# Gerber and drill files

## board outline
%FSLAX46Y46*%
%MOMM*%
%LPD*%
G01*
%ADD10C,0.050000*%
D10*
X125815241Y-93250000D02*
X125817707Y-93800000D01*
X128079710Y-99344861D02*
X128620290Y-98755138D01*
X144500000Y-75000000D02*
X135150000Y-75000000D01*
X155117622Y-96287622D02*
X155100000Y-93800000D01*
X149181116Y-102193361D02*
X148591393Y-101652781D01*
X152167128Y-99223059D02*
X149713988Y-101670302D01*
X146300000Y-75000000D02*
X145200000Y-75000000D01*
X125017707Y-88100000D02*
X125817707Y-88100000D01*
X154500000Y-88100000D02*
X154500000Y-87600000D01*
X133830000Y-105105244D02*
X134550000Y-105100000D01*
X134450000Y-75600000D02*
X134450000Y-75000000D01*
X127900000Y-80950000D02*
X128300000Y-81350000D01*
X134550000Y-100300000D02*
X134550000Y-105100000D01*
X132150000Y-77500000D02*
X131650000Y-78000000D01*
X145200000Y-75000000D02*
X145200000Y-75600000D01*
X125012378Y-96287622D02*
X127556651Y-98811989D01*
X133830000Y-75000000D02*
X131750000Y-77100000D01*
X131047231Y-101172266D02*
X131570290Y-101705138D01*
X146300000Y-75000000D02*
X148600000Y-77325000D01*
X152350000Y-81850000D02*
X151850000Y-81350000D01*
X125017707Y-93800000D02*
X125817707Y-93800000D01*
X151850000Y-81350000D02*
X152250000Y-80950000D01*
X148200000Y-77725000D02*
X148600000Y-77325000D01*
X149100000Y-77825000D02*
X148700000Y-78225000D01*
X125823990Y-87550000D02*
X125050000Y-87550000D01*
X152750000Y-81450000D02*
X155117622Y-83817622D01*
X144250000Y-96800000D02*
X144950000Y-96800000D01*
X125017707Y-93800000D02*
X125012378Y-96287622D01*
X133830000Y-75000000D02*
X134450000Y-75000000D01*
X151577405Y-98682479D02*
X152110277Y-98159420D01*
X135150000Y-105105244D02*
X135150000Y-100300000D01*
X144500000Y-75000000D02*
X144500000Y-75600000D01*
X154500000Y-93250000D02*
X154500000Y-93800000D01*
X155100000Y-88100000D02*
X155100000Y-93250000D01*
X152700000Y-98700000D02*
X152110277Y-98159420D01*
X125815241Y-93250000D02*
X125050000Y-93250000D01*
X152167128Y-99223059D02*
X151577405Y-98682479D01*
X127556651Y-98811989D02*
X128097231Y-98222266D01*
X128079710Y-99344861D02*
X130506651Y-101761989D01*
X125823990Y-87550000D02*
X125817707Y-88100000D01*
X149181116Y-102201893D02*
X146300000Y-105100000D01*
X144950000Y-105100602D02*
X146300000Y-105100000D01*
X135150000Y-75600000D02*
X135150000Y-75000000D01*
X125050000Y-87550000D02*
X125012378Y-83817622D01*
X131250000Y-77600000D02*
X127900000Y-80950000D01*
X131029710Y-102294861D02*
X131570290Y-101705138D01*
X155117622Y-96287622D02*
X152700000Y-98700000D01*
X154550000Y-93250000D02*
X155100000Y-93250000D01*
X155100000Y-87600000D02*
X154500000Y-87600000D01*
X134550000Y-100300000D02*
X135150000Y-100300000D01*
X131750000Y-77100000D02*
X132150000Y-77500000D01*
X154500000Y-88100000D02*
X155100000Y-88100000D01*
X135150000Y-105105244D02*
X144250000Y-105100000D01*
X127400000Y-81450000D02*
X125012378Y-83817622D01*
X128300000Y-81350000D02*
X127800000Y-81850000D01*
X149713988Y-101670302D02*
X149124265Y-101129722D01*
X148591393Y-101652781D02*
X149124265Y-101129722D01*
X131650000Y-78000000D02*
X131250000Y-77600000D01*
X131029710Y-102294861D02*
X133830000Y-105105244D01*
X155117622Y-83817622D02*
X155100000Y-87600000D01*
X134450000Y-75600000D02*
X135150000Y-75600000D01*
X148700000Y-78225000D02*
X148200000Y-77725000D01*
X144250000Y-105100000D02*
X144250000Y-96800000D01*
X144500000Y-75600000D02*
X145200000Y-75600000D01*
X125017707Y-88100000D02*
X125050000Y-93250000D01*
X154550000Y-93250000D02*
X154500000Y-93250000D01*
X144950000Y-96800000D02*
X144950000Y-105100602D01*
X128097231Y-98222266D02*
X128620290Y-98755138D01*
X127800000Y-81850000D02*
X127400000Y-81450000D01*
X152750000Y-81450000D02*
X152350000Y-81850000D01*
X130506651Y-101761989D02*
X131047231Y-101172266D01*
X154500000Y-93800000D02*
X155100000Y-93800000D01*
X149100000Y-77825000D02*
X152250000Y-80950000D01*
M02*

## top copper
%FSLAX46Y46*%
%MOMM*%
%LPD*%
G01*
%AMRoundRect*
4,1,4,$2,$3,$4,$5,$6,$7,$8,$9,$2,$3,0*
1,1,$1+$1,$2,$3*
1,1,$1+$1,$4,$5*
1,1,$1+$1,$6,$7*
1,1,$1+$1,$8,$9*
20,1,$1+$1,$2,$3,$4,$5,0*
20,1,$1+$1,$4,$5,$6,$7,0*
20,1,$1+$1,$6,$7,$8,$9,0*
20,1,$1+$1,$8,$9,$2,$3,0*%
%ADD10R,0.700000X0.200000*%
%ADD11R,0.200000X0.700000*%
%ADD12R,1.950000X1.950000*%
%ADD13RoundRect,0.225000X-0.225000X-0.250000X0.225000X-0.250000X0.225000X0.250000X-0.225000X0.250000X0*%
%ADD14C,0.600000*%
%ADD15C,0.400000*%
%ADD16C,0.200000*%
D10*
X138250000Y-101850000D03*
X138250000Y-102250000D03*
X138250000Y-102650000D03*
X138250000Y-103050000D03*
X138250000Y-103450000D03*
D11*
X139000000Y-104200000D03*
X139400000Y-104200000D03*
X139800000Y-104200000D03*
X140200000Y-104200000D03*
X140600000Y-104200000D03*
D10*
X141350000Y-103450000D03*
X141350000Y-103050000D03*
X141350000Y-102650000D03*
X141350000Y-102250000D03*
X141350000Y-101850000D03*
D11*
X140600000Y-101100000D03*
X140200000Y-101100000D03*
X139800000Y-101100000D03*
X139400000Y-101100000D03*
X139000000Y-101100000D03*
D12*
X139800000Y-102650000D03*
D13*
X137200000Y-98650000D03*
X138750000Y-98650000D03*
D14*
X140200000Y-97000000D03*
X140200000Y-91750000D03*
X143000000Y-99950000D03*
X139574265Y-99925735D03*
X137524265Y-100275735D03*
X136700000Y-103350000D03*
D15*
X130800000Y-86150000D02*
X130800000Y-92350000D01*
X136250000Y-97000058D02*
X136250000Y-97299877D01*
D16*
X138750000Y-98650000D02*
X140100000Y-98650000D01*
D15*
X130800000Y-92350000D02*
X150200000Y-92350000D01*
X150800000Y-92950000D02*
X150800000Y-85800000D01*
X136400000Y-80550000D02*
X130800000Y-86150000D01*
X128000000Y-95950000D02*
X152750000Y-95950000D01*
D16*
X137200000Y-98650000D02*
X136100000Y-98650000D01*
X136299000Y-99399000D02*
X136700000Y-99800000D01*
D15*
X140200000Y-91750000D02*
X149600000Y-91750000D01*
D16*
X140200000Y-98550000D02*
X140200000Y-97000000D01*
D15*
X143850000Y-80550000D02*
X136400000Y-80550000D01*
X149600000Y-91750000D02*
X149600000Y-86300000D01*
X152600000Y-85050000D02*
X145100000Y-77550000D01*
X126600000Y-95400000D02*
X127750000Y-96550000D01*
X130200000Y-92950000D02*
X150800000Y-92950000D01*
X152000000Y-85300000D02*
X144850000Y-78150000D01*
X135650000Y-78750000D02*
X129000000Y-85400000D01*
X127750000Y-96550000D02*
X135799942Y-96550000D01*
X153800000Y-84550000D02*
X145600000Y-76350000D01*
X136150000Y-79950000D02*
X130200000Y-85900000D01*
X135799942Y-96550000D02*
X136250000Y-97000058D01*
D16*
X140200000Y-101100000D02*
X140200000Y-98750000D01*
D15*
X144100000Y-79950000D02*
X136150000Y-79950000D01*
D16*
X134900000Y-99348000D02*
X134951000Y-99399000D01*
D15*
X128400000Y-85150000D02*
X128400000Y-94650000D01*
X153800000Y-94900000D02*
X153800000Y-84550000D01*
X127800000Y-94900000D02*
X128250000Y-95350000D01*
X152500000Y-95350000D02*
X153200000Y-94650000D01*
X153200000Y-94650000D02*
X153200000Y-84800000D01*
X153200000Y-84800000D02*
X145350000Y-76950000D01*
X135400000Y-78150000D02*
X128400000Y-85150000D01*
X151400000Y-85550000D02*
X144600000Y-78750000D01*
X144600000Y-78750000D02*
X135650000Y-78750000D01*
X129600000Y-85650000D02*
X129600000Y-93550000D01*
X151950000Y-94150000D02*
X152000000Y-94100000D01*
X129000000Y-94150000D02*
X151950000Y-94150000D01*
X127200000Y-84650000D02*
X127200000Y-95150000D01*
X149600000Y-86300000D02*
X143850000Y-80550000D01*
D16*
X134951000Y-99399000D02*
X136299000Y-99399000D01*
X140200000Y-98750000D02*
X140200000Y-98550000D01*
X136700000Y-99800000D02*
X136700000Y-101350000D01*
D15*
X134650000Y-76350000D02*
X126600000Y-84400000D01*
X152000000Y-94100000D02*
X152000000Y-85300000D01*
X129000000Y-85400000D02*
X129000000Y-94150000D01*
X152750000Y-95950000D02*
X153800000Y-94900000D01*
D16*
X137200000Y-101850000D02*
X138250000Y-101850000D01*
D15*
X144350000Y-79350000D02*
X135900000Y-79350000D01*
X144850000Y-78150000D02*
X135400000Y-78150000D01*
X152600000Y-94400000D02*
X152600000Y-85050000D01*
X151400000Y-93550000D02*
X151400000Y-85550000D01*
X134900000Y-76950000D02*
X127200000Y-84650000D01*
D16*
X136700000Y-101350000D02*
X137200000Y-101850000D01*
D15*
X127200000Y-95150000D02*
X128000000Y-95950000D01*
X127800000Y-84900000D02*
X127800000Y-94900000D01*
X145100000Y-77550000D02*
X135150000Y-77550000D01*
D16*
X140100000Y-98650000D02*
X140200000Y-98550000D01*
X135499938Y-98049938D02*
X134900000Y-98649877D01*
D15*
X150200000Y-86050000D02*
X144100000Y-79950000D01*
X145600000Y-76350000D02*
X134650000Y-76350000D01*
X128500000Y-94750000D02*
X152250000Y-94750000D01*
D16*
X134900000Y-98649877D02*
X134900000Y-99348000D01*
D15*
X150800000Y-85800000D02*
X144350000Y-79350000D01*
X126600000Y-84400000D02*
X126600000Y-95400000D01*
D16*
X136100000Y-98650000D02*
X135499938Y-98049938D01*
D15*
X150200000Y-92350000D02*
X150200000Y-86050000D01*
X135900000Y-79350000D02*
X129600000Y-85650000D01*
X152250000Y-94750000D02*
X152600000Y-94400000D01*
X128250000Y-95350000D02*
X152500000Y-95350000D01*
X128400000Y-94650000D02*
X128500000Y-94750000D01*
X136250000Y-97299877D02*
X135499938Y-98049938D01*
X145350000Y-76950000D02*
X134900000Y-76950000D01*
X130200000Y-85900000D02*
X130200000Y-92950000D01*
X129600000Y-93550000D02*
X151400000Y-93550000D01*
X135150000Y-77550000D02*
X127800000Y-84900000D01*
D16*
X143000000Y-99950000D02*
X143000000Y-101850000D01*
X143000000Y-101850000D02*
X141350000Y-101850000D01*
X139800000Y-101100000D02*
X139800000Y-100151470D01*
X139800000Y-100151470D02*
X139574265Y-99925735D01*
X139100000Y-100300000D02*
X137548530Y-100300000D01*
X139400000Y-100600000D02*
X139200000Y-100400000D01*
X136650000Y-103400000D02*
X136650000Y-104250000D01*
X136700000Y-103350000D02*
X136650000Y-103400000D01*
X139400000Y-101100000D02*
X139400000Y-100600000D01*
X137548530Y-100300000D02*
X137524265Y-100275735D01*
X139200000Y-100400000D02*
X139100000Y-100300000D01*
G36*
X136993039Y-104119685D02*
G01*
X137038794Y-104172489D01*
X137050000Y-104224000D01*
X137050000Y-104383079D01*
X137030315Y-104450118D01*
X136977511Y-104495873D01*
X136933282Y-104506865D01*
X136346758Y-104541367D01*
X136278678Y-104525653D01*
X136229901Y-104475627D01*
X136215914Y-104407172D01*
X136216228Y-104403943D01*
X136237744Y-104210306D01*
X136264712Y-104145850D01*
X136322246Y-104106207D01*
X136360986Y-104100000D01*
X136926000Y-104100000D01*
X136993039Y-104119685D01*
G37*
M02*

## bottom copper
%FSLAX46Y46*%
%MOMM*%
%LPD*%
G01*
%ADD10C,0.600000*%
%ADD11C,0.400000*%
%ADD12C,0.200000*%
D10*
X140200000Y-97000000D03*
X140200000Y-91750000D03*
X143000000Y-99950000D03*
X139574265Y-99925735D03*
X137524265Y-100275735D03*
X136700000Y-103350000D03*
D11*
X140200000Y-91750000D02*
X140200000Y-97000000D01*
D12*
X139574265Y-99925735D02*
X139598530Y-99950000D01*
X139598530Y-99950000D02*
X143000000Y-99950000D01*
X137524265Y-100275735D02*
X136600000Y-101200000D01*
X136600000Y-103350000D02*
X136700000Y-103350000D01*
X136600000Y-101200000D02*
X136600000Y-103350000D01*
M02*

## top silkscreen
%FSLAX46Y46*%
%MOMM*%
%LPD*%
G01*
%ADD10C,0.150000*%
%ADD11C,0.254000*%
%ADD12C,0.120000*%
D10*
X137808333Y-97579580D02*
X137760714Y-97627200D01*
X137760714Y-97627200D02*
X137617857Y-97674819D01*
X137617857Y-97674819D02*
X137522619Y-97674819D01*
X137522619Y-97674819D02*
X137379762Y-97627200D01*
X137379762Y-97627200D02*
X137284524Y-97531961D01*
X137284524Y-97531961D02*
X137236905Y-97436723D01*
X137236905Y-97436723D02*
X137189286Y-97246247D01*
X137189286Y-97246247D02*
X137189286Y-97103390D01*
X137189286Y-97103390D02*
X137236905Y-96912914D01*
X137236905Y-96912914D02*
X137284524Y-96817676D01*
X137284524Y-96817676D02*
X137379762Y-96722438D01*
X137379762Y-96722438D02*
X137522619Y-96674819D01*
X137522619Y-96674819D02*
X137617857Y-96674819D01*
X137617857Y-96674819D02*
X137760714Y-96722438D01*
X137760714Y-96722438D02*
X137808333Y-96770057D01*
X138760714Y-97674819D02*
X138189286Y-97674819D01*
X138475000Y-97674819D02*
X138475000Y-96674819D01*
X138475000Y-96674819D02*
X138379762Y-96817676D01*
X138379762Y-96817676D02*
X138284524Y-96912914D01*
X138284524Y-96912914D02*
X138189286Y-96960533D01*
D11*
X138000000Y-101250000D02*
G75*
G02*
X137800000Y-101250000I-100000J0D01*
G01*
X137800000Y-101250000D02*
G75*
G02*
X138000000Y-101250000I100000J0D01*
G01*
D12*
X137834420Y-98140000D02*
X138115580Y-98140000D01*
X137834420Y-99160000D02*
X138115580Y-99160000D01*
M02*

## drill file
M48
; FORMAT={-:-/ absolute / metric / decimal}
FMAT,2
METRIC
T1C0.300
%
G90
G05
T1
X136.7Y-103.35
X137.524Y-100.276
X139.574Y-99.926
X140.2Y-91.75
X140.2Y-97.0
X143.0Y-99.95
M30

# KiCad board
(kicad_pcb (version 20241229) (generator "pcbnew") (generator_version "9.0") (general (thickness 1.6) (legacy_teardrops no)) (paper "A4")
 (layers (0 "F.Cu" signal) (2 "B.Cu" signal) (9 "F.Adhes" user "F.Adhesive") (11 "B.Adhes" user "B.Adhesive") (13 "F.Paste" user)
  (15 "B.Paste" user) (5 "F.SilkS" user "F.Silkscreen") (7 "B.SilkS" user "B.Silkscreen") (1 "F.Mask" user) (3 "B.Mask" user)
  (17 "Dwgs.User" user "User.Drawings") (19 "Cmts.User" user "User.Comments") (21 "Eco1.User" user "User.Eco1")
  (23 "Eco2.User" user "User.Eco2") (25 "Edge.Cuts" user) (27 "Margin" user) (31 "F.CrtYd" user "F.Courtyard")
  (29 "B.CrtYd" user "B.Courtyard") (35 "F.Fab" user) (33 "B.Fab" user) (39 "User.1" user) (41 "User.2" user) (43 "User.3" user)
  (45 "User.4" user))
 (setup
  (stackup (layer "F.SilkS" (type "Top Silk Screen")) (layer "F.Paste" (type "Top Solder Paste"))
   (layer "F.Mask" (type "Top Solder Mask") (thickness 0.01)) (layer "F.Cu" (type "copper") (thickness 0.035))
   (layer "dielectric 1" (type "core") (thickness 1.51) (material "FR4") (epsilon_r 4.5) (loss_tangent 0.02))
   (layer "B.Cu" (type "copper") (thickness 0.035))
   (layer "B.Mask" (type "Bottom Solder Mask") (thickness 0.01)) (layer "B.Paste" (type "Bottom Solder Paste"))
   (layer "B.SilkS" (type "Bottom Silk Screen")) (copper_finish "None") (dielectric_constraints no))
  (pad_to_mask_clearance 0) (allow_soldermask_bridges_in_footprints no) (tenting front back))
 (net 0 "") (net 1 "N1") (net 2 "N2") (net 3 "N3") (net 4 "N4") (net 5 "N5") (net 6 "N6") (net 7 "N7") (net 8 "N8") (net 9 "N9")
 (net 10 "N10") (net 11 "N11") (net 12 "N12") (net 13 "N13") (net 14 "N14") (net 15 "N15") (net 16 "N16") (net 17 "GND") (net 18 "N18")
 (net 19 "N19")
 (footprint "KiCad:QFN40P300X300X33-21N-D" (layer "F.Cu") (at 139.8 102.65)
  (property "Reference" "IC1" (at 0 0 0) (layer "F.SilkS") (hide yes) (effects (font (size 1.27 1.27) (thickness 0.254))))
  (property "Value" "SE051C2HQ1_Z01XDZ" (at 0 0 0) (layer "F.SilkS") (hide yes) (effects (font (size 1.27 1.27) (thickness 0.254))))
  (fp_circle (center -1.9 -1.4) (end -1.8 -1.4) (stroke (width 0.254) (type solid)) (fill no) (layer "F.SilkS"))
  (pad "1" smd rect (at -1.55 -0.8 90) (size 0.2 0.7) (layers "F.Cu" "F.Mask" "F.Paste") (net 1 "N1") (solder_mask_margin 0.04)
   (thermal_bridge_angle 45))
  (pad "2" smd rect (at -1.55 -0.4 90) (size 0.2 0.7) (layers "F.Cu" "F.Mask" "F.Paste") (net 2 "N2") (solder_mask_margin 0.04)
   (thermal_bridge_angle 45))
  (pad "3" smd rect (at -1.55 0 90) (size 0.2 0.7) (layers "F.Cu" "F.Mask" "F.Paste") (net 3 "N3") (solder_mask_margin 0.04)
   (thermal_bridge_angle 45))
  (pad "4" smd rect (at -1.55 0.4 90) (size 0.2 0.7) (layers "F.Cu" "F.Mask" "F.Paste") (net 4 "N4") (solder_mask_margin 0.04)
   (thermal_bridge_angle 45))
  (pad "5" smd rect (at -1.55 0.8 90) (size 0.2 0.7) (layers "F.Cu" "F.Mask" "F.Paste") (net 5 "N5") (solder_mask_margin 0.04)
   (thermal_bridge_angle 45))
  (pad "6" smd rect (at -0.8 1.55) (size 0.2 0.7) (layers "F.Cu" "F.Mask" "F.Paste") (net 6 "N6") (solder_mask_margin 0.04)
   (thermal_bridge_angle 45))
  (pad "7" smd rect (at -0.4 1.55) (size 0.2 0.7) (layers "F.Cu" "F.Mask" "F.Paste") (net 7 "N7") (solder_mask_margin 0.04)
   (thermal_bridge_angle 45))
  (pad "8" smd rect (at 0 1.55) (size 0.2 0.7) (layers "F.Cu" "F.Mask" "F.Paste") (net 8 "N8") (solder_mask_margin 0.04)
   (thermal_bridge_angle 45))
  (pad "9" smd rect (at 0.4 1.55) (size 0.2 0.7) (layers "F.Cu" "F.Mask" "F.Paste") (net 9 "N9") (solder_mask_margin 0.04)
   (thermal_bridge_angle 45))
  (pad "10" smd rect (at 0.8 1.55) (size 0.2 0.7) (layers "F.Cu" "F.Mask" "F.Paste") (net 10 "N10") (solder_mask_margin 0.04)
   (thermal_bridge_angle 45))
  (pad "11" smd rect (at 1.55 0.8 90) (size 0.2 0.7) (layers "F.Cu" "F.Mask" "F.Paste") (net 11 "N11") (solder_mask_margin 0.04)
   (thermal_bridge_angle 45))
  (pad "12" smd rect (at 1.55 0.4 90) (size 0.2 0.7) (layers "F.Cu" "F.Mask" "F.Paste") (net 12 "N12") (solder_mask_margin 0.04)
   (thermal_bridge_angle 45))
  (pad "13" smd rect (at 1.55 0 90) (size 0.2 0.7) (layers "F.Cu" "F.Mask" "F.Paste") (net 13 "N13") (solder_mask_margin 0.04)
   (thermal_bridge_angle 45))
  (pad "14" smd rect (at 1.55 -0.4 90) (size 0.2 0.7) (layers "F.Cu" "F.Mask" "F.Paste") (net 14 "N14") (solder_mask_margin 0.04)
   (thermal_bridge_angle 45))
  (pad "15" smd rect (at 1.55 -0.8 90) (size 0.2 0.7) (layers "F.Cu" "F.Mask" "F.Paste") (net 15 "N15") (solder_mask_margin 0.04)
   (thermal_bridge_angle 45))
  (pad "16" smd rect (at 0.8 -1.55) (size 0.2 0.7) (layers "F.Cu" "F.Mask" "F.Paste") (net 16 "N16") (solder_mask_margin 0.04)
   (thermal_bridge_angle 45))
  (pad "17" smd rect (at 0.4 -1.55) (size 0.2 0.7) (layers "F.Cu" "F.Mask" "F.Paste") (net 1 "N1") (solder_mask_margin 0.04)
   (thermal_bridge_angle 45))
  (pad "18" smd rect (at 0 -1.55) (size 0.2 0.7) (layers "F.Cu" "F.Mask" "F.Paste") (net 15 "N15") (solder_mask_margin 0.04)
   (thermal_bridge_angle 45))
  (pad "19" smd rect (at -0.4 -1.55) (size 0.2 0.7) (layers "F.Cu" "F.Mask" "F.Paste") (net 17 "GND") (solder_mask_margin 0.04)
   (thermal_bridge_angle 45))
  (pad "20" smd rect (at -0.8 -1.55) (size 0.2 0.7) (layers "F.Cu" "F.Mask" "F.Paste") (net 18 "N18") (solder_mask_margin 0.04)
   (thermal_bridge_angle 45))
  (pad "21" smd rect (at 0 0) (size 1.95 1.95) (layers "F.Cu" "F.Mask" "F.Paste") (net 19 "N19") (thermal_bridge_angle 45)))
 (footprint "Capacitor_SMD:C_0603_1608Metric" (layer "F.Cu") (at 137.975 98.65)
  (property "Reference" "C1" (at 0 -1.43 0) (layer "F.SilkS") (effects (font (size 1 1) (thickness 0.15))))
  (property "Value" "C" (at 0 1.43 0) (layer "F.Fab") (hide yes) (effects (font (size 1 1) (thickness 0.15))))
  (fp_line (start -0.14058 -0.51) (end 0.14058 -0.51) (stroke (width 0.12) (type solid)) (layer "F.SilkS"))
  (fp_line (start -0.14058 0.51) (end 0.14058 0.51) (stroke (width 0.12) (type solid)) (layer "F.SilkS"))
  (pad "1" smd roundrect (at -0.775 0) (size 0.9 0.95) (layers "F.Cu" "F.Mask" "F.Paste") (roundrect_rratio 0.25) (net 1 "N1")
   (solder_mask_margin 0.04))
  (pad "2" smd roundrect (at 0.775 0) (size 0.9 0.95) (layers "F.Cu" "F.Mask" "F.Paste") (roundrect_rratio 0.25) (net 1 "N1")
   (solder_mask_margin 0.04)))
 (gr_line (start 125.815241 93.25) (end 125.817707 93.8) (stroke (width 0.05) (type default)) (layer "Edge.Cuts"))
 (gr_line (start 128.07971 99.344861) (end 128.62029 98.755138) (stroke (width 0.05) (type solid)) (layer "Edge.Cuts"))
 (gr_line (start 144.5 75) (end 135.15 75) (stroke (width 0.05) (type default)) (layer "Edge.Cuts"))
 (gr_line (start 155.117622 96.287622) (end 155.1 93.8) (stroke (width 0.05) (type default)) (layer "Edge.Cuts"))
 (gr_line (start 149.181116 102.193361) (end 148.591393 101.652781) (stroke (width 0.05) (type solid)) (layer "Edge.Cuts"))
 (gr_line (start 152.167128 99.223059) (end 149.713988 101.670302) (stroke (width 0.05) (type default)) (layer "Edge.Cuts"))
 (gr_line (start 146.3 75) (end 145.2 75) (stroke (width 0.05) (type default)) (layer "Edge.Cuts"))
 (gr_line (start 125.017707 88.1) (end 125.817707 88.1) (stroke (width 0.05) (type solid)) (layer "Edge.Cuts"))
 (gr_line (start 154.5 88.1) (end 154.5 87.6) (stroke (width 0.05) (type default)) (layer "Edge.Cuts"))
 (gr_line (start 133.83 105.105244) (end 134.55 105.1) (stroke (width 0.05) (type default)) (layer "Edge.Cuts"))
 (gr_line (start 134.45 75.6) (end 134.45 75) (stroke (width 0.05) (type solid)) (layer "Edge.Cuts"))
 (gr_line (start 127.9 80.95) (end 128.3 81.35) (stroke (width 0.05) (type default)) (layer "Edge.Cuts"))
 (gr_line (start 134.55 100.3) (end 134.55 105.1) (stroke (width 0.05) (type solid)) (layer "Edge.Cuts"))
 (gr_line (start 132.15 77.5) (end 131.65 78) (stroke (width 0.05) (type default)) (layer "Edge.Cuts"))
 (gr_line (start 145.2 75) (end 145.2 75.6) (stroke (width 0.05) (type solid)) (layer "Edge.Cuts"))
 (gr_line (start 125.012378 96.287622) (end 127.556651 98.811989) (stroke (width 0.05) (type default)) (layer "Edge.Cuts"))
 (gr_line (start 133.83 75) (end 131.75 77.1) (stroke (width 0.05) (type default)) (layer "Edge.Cuts"))
 (gr_line (start 131.047231 101.172266) (end 131.57029 101.705138) (stroke (width 0.05) (type default)) (layer "Edge.Cuts"))
 (gr_line (start 146.3 75) (end 148.6 77.325) (stroke (width 0.05) (type default)) (layer "Edge.Cuts"))
 (gr_line (start 152.35 81.85) (end 151.85 81.35) (stroke (width 0.05) (type default)) (layer "Edge.Cuts"))
 (gr_line (start 125.017707 93.8) (end 125.817707 93.8) (stroke (width 0.05) (type solid)) (layer "Edge.Cuts"))
 (gr_line (start 151.85 81.35) (end 152.25 80.95) (stroke (width 0.05) (type default)) (layer "Edge.Cuts"))
 (gr_line (start 148.2 77.725) (end 148.6 77.325) (stroke (width 0.05) (type default)) (layer "Edge.Cuts"))
 (gr_line (start 149.1 77.825) (end 148.7 78.225) (stroke (width 0.05) (type default)) (layer "Edge.Cuts"))
 (gr_line (start 125.82399 87.55) (end 125.05 87.55) (stroke (width 0.05) (type solid)) (layer "Edge.Cuts"))
 (gr_line (start 152.75 81.45) (end 155.117622 83.817622) (stroke (width 0.05) (type default)) (layer "Edge.Cuts"))
 (gr_line (start 144.25 96.8) (end 144.95 96.8) (stroke (width 0.05) (type default)) (layer "Edge.Cuts"))
 (gr_line (start 125.017707 93.8) (end 125.012378 96.287622) (stroke (width 0.05) (type default)) (layer "Edge.Cuts"))
 (gr_line (start 133.83 75) (end 134.45 75) (stroke (width 0.05) (type default)) (layer "Edge.Cuts"))
 (gr_line (start 151.577405 98.682479) (end 152.110277 98.15942) (stroke (width 0.05) (type default)) (layer "Edge.Cuts"))
 (gr_line (start 135.15 105.105244) (end 135.15 100.3) (stroke (width 0.05) (type default)) (layer "Edge.Cuts"))
 (gr_line (start 144.5 75) (end 144.5 75.6) (stroke (width 0.05) (type solid)) (layer "Edge.Cuts"))
 (gr_line (start 154.5 93.25) (end 154.5 93.8) (stroke (width 0.05) (type default)) (layer "Edge.Cuts"))
 (gr_line (start 155.1 88.1) (end 155.1 93.25) (stroke (width 0.05) (type default)) (layer "Edge.Cuts"))
 (gr_line (start 152.7 98.7) (end 152.110277 98.15942) (stroke (width 0.05) (type solid)) (layer "Edge.Cuts"))
 (gr_line (start 125.815241 93.25) (end 125.05 93.25) (stroke (width 0.05) (type solid)) (layer "Edge.Cuts"))
 (gr_line (start 152.167128 99.223059) (end 151.577405 98.682479) (stroke (width 0.05) (type solid)) (layer "Edge.Cuts"))
 (gr_line (start 127.556651 98.811989) (end 128.097231 98.222266) (stroke (width 0.05) (type solid)) (layer "Edge.Cuts"))
 (gr_line (start 128.07971 99.344861) (end 130.506651 101.761989) (stroke (width 0.05) (type default)) (layer "Edge.Cuts"))
 (gr_line (start 125.82399 87.55) (end 125.817707 88.1) (stroke (width 0.05) (type default)) (layer "Edge.Cuts"))
 (gr_line (start 149.181116 102.201893) (end 146.3 105.1) (stroke (width 0.05) (type default)) (layer "Edge.Cuts"))
 (gr_line (start 144.95 105.100602) (end 146.3 105.1) (stroke (width 0.05) (type default)) (layer "Edge.Cuts"))
 (gr_line (start 135.15 75.6) (end 135.15 75) (stroke (width 0.05) (type solid)) (layer "Edge.Cuts"))
 (gr_line (start 125.05 87.55) (end 125.012378 83.817622) (stroke (width 0.05) (type default)) (layer "Edge.Cuts"))
 (gr_line (start 131.25 77.6) (end 127.9 80.95) (stroke (width 0.05) (type default)) (layer "Edge.Cuts"))
 (gr_line (start 131.02971 102.294861) (end 131.57029 101.705138) (stroke (width 0.05) (type solid)) (layer "Edge.Cuts"))
 (gr_line (start 155.117622 96.287622) (end 152.7 98.7) (stroke (width 0.05) (type default)) (layer "Edge.Cuts"))
 (gr_line (start 154.55 93.25) (end 155.1 93.25) (stroke (width 0.05) (type default)) (layer "Edge.Cuts"))
 (gr_line (start 155.1 87.6) (end 154.5 87.6) (stroke (width 0.05) (type default)) (layer "Edge.Cuts"))
 (gr_line (start 134.55 100.3) (end 135.15 100.3) (stroke (width 0.05) (type default)) (layer "Edge.Cuts"))
 (gr_line (start 131.75 77.1) (end 132.15 77.5) (stroke (width 0.05) (type default)) (layer "Edge.Cuts"))
 (gr_line (start 154.5 88.1) (end 155.1 88.1) (stroke (width 0.05) (type default)) (layer "Edge.Cuts"))
 (gr_line (start 135.15 105.105244) (end 144.25 105.1) (stroke (width 0.05) (type default)) (layer "Edge.Cuts"))
 (gr_line (start 127.4 81.45) (end 125.012378 83.817622) (stroke (width 0.05) (type default)) (layer "Edge.Cuts"))
 (gr_line (start 128.3 81.35) (end 127.8 81.85) (stroke (width 0.05) (type default)) (layer "Edge.Cuts"))
 (gr_line (start 149.713988 101.670302) (end 149.124265 101.129722) (stroke (width 0.05) (type solid)) (layer "Edge.Cuts"))
 (gr_line (start 148.591393 101.652781) (end 149.124265 101.129722) (stroke (width 0.05) (type default)) (layer "Edge.Cuts"))
 (gr_line (start 131.65 78) (end 131.25 77.6) (stroke (width 0.05) (type default)) (layer "Edge.Cuts"))
 (gr_line (start 131.02971 102.294861) (end 133.83 105.105244) (stroke (width 0.05) (type default)) (layer "Edge.Cuts"))
 (gr_line (start 155.117622 83.817622) (end 155.1 87.6) (stroke (width 0.05) (type default)) (layer "Edge.Cuts"))
 (gr_line (start 134.45 75.6) (end 135.15 75.6) (stroke (width 0.05) (type default)) (layer "Edge.Cuts"))
 (gr_line (start 148.7 78.225) (end 148.2 77.725) (stroke (width 0.05) (type default)) (layer "Edge.Cuts"))
 (gr_line (start 144.25 105.1) (end 144.25 96.8) (stroke (width 0.05) (type default)) (layer "Edge.Cuts"))
 (gr_line (start 144.5 75.6) (end 145.2 75.6) (stroke (width 0.05) (type default)) (layer "Edge.Cuts"))
 (gr_line (start 125.017707 88.1) (end 125.05 93.25) (stroke (width 0.05) (type default)) (layer "Edge.Cuts"))
 (gr_line (start 154.55 93.25) (end 154.5 93.25) (stroke (width 0.05) (type default)) (layer "Edge.Cuts"))
 (gr_line (start 144.95 96.8) (end 144.95 105.100602) (stroke (width 0.05) (type solid)) (layer "Edge.Cuts"))
 (gr_line (start 128.097231 98.222266) (end 128.62029 98.755138) (stroke (width 0.05) (type default)) (layer "Edge.Cuts"))
 (gr_line (start 127.8 81.85) (end 127.4 81.45) (stroke (width 0.05) (type default)) (layer "Edge.Cuts"))
 (gr_line (start 152.75 81.45) (end 152.35 81.85) (stroke (width 0.05) (type default)) (layer "Edge.Cuts"))
 (gr_line (start 130.506651 101.761989) (end 131.047231 101.172266) (stroke (width 0.05) (type solid)) (layer "Edge.Cuts"))
 (gr_line (start 154.5 93.8) (end 155.1 93.8) (stroke (width 0.05) (type default)) (layer "Edge.Cuts"))
 (gr_line (start 149.1 77.825) (end 152.25 80.95) (stroke (width 0.05) (type default)) (layer "Edge.Cuts"))
 (segment (start 130.8 86.15) (end 130.8 92.35) (width 0.4) (layer "F.Cu") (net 1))
 (segment (start 136.25 97.000058) (end 136.25 97.299877) (width 0.4) (layer "F.Cu") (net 1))
 (segment (start 138.75 98.65) (end 140.1 98.65) (width 0.2) (layer "F.Cu") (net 1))
 (segment (start 130.8 92.35) (end 150.2 92.35) (width 0.4) (layer "F.Cu") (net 1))
 (segment (start 150.8 92.95) (end 150.8 85.8) (width 0.4) (layer "F.Cu") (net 1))
 (segment (start 136.4 80.55) (end 130.8 86.15) (width 0.4) (layer "F.Cu") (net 1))
 (segment (start 128 95.95) (end 152.75 95.95) (width 0.4) (layer "F.Cu") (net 1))
 (segment (start 137.2 98.65) (end 136.1 98.65) (width 0.2) (layer "F.Cu") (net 1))
 (segment (start 136.299 99.399) (end 136.7 99.8) (width 0.2) (layer "F.Cu") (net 1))
 (segment (start 140.2 91.75) (end 149.6 91.75) (width 0.4) (layer "F.Cu") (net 1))
 (segment (start 140.2 98.55) (end 140.2 97) (width 0.2) (layer "F.Cu") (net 1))
 (segment (start 143.85 80.55) (end 136.4 80.55) (width 0.4) (layer "F.Cu") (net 1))
 (segment (start 149.6 91.75) (end 149.6 86.3) (width 0.4) (layer "F.Cu") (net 1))
 (segment (start 152.6 85.05) (end 145.1 77.55) (width 0.4) (layer "F.Cu") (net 1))
 (segment (start 126.6 95.4) (end 127.75 96.55) (width 0.4) (layer "F.Cu") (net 1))
 (segment (start 130.2 92.95) (end 150.8 92.95) (width 0.4) (layer "F.Cu") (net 1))
 (segment (start 152 85.3) (end 144.85 78.15) (width 0.4) (layer "F.Cu") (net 1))
 (segment (start 135.65 78.75) (end 129 85.4) (width 0.4) (layer "F.Cu") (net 1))
 (segment (start 127.75 96.55) (end 135.799942 96.55) (width 0.4) (layer "F.Cu") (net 1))
 (segment (start 153.8 84.55) (end 145.6 76.35) (width 0.4) (layer "F.Cu") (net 1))
 (segment (start 136.15 79.95) (end 130.2 85.9) (width 0.4) (layer "F.Cu") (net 1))
 (segment (start 135.799942 96.55) (end 136.25 97.000058) (width 0.4) (layer "F.Cu") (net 1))
 (segment (start 140.2 101.1) (end 140.2 98.75) (width 0.2) (layer "F.Cu") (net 1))
 (segment (start 144.1 79.95) (end 136.15 79.95) (width 0.4) (layer "F.Cu") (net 1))
 (segment (start 134.9 99.348) (end 134.951 99.399) (width 0.2) (layer "F.Cu") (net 1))
 (segment (start 128.4 85.15) (end 128.4 94.65) (width 0.4) (layer "F.Cu") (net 1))
 (segment (start 153.8 94.9) (end 153.8 84.55) (width 0.4) (layer "F.Cu") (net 1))
 (segment (start 127.8 94.9) (end 128.25 95.35) (width 0.4) (layer "F.Cu") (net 1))
 (segment (start 152.5 95.35) (end 153.2 94.65) (width 0.4) (layer "F.Cu") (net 1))
 (segment (start 153.2 94.65) (end 153.2 84.8) (width 0.4) (layer "F.Cu") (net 1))
 (segment (start 153.2 84.8) (end 145.35 76.95) (width 0.4) (layer "F.Cu") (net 1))
 (segment (start 135.4 78.15) (end 128.4 85.15) (width 0.4) (layer "F.Cu") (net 1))
 (segment (start 151.4 85.55) (end 144.6 78.75) (width 0.4) (layer "F.Cu") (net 1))
 (segment (start 144.6 78.75) (end 135.65 78.75) (width 0.4) (layer "F.Cu") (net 1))
 (segment (start 129.6 85.65) (end 129.6 93.55) (width 0.4) (layer "F.Cu") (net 1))
 (segment (start 151.95 94.15) (end 152 94.1) (width 0.4) (layer "F.Cu") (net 1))
 (segment (start 129 94.15) (end 151.95 94.15) (width 0.4) (layer "F.Cu") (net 1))
 (segment (start 127.2 84.65) (end 127.2 95.15) (width 0.4) (layer "F.Cu") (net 1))
 (segment (start 149.6 86.3) (end 143.85 80.55) (width 0.4) (layer "F.Cu") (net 1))
 (segment (start 134.951 99.399) (end 136.299 99.399) (width 0.2) (layer "F.Cu") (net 1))
 (segment (start 140.2 98.75) (end 140.2 98.55) (width 0.2) (layer "F.Cu") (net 1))
 (segment (start 136.7 99.8) (end 136.7 101.35) (width 0.2) (layer "F.Cu") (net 1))
 (segment (start 134.65 76.35) (end 126.6 84.4) (width 0.4) (layer "F.Cu") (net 1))
 (segment (start 152 94.1) (end 152 85.3) (width 0.4) (layer "F.Cu") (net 1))
 (segment (start 129 85.4) (end 129 94.15) (width 0.4) (layer "F.Cu") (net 1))
 (segment (start 152.75 95.95) (end 153.8 94.9) (width 0.4) (layer "F.Cu") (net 1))
 (segment (start 137.2 101.85) (end 138.25 101.85) (width 0.2) (layer "F.Cu") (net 1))
 (segment (start 144.35 79.35) (end 135.9 79.35) (width 0.4) (layer "F.Cu") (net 1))
 (segment (start 144.85 78.15) (end 135.4 78.15) (width 0.4) (layer "F.Cu") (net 1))
 (segment (start 152.6 94.4) (end 152.6 85.05) (width 0.4) (layer "F.Cu") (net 1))
 (segment (start 151.4 93.55) (end 151.4 85.55) (width 0.4) (layer "F.Cu") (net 1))
 (segment (start 134.9 76.95) (end 127.2 84.65) (width 0.4) (layer "F.Cu") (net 1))
 (segment (start 136.7 101.35) (end 137.2 101.85) (width 0.2) (layer "F.Cu") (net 1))
 (segment (start 127.2 95.15) (end 128 95.95) (width 0.4) (layer "F.Cu") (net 1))
 (segment (start 127.8 84.9) (end 127.8 94.9) (width 0.4) (layer "F.Cu") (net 1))
 (segment (start 145.1 77.55) (end 135.15 77.55) (width 0.4) (layer "F.Cu") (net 1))
 (segment (start 140.1 98.65) (end 140.2 98.55) (width 0.2) (layer "F.Cu") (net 1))
 (segment (start 135.499938 98.049938) (end 134.9 98.649877) (width 0.2) (layer "F.Cu") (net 1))
 (segment (start 150.2 86.05) (end 144.1 79.95) (width 0.4) (layer "F.Cu") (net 1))
 (segment (start 145.6 76.35) (end 134.65 76.35) (width 0.4) (layer "F.Cu") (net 1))
 (segment (start 128.5 94.75) (end 152.25 94.75) (width 0.4) (layer "F.Cu") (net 1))
 (segment (start 134.9 98.649877) (end 134.9 99.348) (width 0.2) (layer "F.Cu") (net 1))
 (segment (start 150.8 85.8) (end 144.35 79.35) (width 0.4) (layer "F.Cu") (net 1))
 (segment (start 126.6 84.4) (end 126.6 95.4) (width 0.4) (layer "F.Cu") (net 1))
 (segment (start 136.1 98.65) (end 135.499938 98.049938) (width 0.2) (layer "F.Cu") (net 1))
 (segment (start 150.2 92.35) (end 150.2 86.05) (width 0.4) (layer "F.Cu") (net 1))
 (segment (start 135.9 79.35) (end 129.6 85.65) (width 0.4) (layer "F.Cu") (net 1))
 (segment (start 152.25 94.75) (end 152.6 94.4) (width 0.4) (layer "F.Cu") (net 1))
 (segment (start 128.25 95.35) (end 152.5 95.35) (width 0.4) (layer "F.Cu") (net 1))
 (segment (start 128.4 94.65) (end 128.5 94.75) (width 0.4) (layer "F.Cu") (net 1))
 (segment (start 136.25 97.299877) (end 135.499938 98.049938) (width 0.4) (layer "F.Cu") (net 1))
 (segment (start 145.35 76.95) (end 134.9 76.95) (width 0.4) (layer "F.Cu") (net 1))
 (segment (start 130.2 85.9) (end 130.2 92.95) (width 0.4) (layer "F.Cu") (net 1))
 (segment (start 129.6 93.55) (end 151.4 93.55) (width 0.4) (layer "F.Cu") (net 1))
 (segment (start 135.15 77.55) (end 127.8 84.9) (width 0.4) (layer "F.Cu") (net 1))
 (via (at 140.2 97) (size 0.6) (drill 0.3) (layers "F.Cu" "B.Cu") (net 1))
 (via (at 140.2 91.75) (size 0.6) (drill 0.3) (layers "F.Cu" "B.Cu") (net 1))
 (segment (start 140.2 91.75) (end 140.2 97) (width 0.4) (layer "B.Cu") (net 1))
 (segment (start 143 99.95) (end 143 101.85) (width 0.2) (layer "F.Cu") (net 15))
 (segment (start 143 101.85) (end 141.35 101.85) (width 0.2) (layer "F.Cu") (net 15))
 (segment (start 139.8 101.1) (end 139.8 100.15147) (width 0.2) (layer "F.Cu") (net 15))
 (segment (start 139.8 100.15147) (end 139.574265 99.925735) (width 0.2) (layer "F.Cu") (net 15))
 (via (at 143 99.95) (size 0.6) (drill 0.3) (layers "F.Cu" "B.Cu") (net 15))
 (via (at 139.574265 99.925735) (size 0.6) (drill 0.3) (layers "F.Cu" "B.Cu") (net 15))
 (segment (start 139.574265 99.925735) (end 139.59853 99.95) (width 0.2) (layer "B.Cu") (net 15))
 (segment (start 139.59853 99.95) (end 143 99.95) (width 0.2) (layer "B.Cu") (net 15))
 (segment (start 139.1 100.3) (end 137.54853 100.3) (width 0.2) (layer "F.Cu") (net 17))
 (segment (start 139.4 100.6) (end 139.2 100.4) (width 0.2) (layer "F.Cu") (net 17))
 (segment (start 136.65 103.4) (end 136.65 104.25) (width 0.2) (layer "F.Cu") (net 17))
 (segment (start 136.7 103.35) (end 136.65 103.4) (width 0.2) (layer "F.Cu") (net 17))
 (segment (start 139.4 101.1) (end 139.4 100.6) (width 0.2) (layer "F.Cu") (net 17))
 (segment (start 137.54853 100.3) (end 137.524265 100.275735) (width 0.2) (layer "F.Cu") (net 17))
 (segment (start 139.2 100.4) (end 139.1 100.3) (width 0.2) (layer "F.Cu") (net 17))
 (via (at 137.524265 100.275735) (size 0.6) (drill 0.3) (layers "F.Cu" "B.Cu") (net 17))
 (via (at 136.7 103.35) (size 0.6) (drill 0.3) (layers "F.Cu" "B.Cu") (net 17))
 (segment (start 137.524265 100.275735) (end 136.6 101.2) (width 0.2) (layer "B.Cu") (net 17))
 (segment (start 136.6 103.35) (end 136.7 103.35) (width 0.2) (layer "B.Cu") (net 17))
 (segment (start 136.6 101.2) (end 136.6 103.35) (width 0.2) (layer "B.Cu") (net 17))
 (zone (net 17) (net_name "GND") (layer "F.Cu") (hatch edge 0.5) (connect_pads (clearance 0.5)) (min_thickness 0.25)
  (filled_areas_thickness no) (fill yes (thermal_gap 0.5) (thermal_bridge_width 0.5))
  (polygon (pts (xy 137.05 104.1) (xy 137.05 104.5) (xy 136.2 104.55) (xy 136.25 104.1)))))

